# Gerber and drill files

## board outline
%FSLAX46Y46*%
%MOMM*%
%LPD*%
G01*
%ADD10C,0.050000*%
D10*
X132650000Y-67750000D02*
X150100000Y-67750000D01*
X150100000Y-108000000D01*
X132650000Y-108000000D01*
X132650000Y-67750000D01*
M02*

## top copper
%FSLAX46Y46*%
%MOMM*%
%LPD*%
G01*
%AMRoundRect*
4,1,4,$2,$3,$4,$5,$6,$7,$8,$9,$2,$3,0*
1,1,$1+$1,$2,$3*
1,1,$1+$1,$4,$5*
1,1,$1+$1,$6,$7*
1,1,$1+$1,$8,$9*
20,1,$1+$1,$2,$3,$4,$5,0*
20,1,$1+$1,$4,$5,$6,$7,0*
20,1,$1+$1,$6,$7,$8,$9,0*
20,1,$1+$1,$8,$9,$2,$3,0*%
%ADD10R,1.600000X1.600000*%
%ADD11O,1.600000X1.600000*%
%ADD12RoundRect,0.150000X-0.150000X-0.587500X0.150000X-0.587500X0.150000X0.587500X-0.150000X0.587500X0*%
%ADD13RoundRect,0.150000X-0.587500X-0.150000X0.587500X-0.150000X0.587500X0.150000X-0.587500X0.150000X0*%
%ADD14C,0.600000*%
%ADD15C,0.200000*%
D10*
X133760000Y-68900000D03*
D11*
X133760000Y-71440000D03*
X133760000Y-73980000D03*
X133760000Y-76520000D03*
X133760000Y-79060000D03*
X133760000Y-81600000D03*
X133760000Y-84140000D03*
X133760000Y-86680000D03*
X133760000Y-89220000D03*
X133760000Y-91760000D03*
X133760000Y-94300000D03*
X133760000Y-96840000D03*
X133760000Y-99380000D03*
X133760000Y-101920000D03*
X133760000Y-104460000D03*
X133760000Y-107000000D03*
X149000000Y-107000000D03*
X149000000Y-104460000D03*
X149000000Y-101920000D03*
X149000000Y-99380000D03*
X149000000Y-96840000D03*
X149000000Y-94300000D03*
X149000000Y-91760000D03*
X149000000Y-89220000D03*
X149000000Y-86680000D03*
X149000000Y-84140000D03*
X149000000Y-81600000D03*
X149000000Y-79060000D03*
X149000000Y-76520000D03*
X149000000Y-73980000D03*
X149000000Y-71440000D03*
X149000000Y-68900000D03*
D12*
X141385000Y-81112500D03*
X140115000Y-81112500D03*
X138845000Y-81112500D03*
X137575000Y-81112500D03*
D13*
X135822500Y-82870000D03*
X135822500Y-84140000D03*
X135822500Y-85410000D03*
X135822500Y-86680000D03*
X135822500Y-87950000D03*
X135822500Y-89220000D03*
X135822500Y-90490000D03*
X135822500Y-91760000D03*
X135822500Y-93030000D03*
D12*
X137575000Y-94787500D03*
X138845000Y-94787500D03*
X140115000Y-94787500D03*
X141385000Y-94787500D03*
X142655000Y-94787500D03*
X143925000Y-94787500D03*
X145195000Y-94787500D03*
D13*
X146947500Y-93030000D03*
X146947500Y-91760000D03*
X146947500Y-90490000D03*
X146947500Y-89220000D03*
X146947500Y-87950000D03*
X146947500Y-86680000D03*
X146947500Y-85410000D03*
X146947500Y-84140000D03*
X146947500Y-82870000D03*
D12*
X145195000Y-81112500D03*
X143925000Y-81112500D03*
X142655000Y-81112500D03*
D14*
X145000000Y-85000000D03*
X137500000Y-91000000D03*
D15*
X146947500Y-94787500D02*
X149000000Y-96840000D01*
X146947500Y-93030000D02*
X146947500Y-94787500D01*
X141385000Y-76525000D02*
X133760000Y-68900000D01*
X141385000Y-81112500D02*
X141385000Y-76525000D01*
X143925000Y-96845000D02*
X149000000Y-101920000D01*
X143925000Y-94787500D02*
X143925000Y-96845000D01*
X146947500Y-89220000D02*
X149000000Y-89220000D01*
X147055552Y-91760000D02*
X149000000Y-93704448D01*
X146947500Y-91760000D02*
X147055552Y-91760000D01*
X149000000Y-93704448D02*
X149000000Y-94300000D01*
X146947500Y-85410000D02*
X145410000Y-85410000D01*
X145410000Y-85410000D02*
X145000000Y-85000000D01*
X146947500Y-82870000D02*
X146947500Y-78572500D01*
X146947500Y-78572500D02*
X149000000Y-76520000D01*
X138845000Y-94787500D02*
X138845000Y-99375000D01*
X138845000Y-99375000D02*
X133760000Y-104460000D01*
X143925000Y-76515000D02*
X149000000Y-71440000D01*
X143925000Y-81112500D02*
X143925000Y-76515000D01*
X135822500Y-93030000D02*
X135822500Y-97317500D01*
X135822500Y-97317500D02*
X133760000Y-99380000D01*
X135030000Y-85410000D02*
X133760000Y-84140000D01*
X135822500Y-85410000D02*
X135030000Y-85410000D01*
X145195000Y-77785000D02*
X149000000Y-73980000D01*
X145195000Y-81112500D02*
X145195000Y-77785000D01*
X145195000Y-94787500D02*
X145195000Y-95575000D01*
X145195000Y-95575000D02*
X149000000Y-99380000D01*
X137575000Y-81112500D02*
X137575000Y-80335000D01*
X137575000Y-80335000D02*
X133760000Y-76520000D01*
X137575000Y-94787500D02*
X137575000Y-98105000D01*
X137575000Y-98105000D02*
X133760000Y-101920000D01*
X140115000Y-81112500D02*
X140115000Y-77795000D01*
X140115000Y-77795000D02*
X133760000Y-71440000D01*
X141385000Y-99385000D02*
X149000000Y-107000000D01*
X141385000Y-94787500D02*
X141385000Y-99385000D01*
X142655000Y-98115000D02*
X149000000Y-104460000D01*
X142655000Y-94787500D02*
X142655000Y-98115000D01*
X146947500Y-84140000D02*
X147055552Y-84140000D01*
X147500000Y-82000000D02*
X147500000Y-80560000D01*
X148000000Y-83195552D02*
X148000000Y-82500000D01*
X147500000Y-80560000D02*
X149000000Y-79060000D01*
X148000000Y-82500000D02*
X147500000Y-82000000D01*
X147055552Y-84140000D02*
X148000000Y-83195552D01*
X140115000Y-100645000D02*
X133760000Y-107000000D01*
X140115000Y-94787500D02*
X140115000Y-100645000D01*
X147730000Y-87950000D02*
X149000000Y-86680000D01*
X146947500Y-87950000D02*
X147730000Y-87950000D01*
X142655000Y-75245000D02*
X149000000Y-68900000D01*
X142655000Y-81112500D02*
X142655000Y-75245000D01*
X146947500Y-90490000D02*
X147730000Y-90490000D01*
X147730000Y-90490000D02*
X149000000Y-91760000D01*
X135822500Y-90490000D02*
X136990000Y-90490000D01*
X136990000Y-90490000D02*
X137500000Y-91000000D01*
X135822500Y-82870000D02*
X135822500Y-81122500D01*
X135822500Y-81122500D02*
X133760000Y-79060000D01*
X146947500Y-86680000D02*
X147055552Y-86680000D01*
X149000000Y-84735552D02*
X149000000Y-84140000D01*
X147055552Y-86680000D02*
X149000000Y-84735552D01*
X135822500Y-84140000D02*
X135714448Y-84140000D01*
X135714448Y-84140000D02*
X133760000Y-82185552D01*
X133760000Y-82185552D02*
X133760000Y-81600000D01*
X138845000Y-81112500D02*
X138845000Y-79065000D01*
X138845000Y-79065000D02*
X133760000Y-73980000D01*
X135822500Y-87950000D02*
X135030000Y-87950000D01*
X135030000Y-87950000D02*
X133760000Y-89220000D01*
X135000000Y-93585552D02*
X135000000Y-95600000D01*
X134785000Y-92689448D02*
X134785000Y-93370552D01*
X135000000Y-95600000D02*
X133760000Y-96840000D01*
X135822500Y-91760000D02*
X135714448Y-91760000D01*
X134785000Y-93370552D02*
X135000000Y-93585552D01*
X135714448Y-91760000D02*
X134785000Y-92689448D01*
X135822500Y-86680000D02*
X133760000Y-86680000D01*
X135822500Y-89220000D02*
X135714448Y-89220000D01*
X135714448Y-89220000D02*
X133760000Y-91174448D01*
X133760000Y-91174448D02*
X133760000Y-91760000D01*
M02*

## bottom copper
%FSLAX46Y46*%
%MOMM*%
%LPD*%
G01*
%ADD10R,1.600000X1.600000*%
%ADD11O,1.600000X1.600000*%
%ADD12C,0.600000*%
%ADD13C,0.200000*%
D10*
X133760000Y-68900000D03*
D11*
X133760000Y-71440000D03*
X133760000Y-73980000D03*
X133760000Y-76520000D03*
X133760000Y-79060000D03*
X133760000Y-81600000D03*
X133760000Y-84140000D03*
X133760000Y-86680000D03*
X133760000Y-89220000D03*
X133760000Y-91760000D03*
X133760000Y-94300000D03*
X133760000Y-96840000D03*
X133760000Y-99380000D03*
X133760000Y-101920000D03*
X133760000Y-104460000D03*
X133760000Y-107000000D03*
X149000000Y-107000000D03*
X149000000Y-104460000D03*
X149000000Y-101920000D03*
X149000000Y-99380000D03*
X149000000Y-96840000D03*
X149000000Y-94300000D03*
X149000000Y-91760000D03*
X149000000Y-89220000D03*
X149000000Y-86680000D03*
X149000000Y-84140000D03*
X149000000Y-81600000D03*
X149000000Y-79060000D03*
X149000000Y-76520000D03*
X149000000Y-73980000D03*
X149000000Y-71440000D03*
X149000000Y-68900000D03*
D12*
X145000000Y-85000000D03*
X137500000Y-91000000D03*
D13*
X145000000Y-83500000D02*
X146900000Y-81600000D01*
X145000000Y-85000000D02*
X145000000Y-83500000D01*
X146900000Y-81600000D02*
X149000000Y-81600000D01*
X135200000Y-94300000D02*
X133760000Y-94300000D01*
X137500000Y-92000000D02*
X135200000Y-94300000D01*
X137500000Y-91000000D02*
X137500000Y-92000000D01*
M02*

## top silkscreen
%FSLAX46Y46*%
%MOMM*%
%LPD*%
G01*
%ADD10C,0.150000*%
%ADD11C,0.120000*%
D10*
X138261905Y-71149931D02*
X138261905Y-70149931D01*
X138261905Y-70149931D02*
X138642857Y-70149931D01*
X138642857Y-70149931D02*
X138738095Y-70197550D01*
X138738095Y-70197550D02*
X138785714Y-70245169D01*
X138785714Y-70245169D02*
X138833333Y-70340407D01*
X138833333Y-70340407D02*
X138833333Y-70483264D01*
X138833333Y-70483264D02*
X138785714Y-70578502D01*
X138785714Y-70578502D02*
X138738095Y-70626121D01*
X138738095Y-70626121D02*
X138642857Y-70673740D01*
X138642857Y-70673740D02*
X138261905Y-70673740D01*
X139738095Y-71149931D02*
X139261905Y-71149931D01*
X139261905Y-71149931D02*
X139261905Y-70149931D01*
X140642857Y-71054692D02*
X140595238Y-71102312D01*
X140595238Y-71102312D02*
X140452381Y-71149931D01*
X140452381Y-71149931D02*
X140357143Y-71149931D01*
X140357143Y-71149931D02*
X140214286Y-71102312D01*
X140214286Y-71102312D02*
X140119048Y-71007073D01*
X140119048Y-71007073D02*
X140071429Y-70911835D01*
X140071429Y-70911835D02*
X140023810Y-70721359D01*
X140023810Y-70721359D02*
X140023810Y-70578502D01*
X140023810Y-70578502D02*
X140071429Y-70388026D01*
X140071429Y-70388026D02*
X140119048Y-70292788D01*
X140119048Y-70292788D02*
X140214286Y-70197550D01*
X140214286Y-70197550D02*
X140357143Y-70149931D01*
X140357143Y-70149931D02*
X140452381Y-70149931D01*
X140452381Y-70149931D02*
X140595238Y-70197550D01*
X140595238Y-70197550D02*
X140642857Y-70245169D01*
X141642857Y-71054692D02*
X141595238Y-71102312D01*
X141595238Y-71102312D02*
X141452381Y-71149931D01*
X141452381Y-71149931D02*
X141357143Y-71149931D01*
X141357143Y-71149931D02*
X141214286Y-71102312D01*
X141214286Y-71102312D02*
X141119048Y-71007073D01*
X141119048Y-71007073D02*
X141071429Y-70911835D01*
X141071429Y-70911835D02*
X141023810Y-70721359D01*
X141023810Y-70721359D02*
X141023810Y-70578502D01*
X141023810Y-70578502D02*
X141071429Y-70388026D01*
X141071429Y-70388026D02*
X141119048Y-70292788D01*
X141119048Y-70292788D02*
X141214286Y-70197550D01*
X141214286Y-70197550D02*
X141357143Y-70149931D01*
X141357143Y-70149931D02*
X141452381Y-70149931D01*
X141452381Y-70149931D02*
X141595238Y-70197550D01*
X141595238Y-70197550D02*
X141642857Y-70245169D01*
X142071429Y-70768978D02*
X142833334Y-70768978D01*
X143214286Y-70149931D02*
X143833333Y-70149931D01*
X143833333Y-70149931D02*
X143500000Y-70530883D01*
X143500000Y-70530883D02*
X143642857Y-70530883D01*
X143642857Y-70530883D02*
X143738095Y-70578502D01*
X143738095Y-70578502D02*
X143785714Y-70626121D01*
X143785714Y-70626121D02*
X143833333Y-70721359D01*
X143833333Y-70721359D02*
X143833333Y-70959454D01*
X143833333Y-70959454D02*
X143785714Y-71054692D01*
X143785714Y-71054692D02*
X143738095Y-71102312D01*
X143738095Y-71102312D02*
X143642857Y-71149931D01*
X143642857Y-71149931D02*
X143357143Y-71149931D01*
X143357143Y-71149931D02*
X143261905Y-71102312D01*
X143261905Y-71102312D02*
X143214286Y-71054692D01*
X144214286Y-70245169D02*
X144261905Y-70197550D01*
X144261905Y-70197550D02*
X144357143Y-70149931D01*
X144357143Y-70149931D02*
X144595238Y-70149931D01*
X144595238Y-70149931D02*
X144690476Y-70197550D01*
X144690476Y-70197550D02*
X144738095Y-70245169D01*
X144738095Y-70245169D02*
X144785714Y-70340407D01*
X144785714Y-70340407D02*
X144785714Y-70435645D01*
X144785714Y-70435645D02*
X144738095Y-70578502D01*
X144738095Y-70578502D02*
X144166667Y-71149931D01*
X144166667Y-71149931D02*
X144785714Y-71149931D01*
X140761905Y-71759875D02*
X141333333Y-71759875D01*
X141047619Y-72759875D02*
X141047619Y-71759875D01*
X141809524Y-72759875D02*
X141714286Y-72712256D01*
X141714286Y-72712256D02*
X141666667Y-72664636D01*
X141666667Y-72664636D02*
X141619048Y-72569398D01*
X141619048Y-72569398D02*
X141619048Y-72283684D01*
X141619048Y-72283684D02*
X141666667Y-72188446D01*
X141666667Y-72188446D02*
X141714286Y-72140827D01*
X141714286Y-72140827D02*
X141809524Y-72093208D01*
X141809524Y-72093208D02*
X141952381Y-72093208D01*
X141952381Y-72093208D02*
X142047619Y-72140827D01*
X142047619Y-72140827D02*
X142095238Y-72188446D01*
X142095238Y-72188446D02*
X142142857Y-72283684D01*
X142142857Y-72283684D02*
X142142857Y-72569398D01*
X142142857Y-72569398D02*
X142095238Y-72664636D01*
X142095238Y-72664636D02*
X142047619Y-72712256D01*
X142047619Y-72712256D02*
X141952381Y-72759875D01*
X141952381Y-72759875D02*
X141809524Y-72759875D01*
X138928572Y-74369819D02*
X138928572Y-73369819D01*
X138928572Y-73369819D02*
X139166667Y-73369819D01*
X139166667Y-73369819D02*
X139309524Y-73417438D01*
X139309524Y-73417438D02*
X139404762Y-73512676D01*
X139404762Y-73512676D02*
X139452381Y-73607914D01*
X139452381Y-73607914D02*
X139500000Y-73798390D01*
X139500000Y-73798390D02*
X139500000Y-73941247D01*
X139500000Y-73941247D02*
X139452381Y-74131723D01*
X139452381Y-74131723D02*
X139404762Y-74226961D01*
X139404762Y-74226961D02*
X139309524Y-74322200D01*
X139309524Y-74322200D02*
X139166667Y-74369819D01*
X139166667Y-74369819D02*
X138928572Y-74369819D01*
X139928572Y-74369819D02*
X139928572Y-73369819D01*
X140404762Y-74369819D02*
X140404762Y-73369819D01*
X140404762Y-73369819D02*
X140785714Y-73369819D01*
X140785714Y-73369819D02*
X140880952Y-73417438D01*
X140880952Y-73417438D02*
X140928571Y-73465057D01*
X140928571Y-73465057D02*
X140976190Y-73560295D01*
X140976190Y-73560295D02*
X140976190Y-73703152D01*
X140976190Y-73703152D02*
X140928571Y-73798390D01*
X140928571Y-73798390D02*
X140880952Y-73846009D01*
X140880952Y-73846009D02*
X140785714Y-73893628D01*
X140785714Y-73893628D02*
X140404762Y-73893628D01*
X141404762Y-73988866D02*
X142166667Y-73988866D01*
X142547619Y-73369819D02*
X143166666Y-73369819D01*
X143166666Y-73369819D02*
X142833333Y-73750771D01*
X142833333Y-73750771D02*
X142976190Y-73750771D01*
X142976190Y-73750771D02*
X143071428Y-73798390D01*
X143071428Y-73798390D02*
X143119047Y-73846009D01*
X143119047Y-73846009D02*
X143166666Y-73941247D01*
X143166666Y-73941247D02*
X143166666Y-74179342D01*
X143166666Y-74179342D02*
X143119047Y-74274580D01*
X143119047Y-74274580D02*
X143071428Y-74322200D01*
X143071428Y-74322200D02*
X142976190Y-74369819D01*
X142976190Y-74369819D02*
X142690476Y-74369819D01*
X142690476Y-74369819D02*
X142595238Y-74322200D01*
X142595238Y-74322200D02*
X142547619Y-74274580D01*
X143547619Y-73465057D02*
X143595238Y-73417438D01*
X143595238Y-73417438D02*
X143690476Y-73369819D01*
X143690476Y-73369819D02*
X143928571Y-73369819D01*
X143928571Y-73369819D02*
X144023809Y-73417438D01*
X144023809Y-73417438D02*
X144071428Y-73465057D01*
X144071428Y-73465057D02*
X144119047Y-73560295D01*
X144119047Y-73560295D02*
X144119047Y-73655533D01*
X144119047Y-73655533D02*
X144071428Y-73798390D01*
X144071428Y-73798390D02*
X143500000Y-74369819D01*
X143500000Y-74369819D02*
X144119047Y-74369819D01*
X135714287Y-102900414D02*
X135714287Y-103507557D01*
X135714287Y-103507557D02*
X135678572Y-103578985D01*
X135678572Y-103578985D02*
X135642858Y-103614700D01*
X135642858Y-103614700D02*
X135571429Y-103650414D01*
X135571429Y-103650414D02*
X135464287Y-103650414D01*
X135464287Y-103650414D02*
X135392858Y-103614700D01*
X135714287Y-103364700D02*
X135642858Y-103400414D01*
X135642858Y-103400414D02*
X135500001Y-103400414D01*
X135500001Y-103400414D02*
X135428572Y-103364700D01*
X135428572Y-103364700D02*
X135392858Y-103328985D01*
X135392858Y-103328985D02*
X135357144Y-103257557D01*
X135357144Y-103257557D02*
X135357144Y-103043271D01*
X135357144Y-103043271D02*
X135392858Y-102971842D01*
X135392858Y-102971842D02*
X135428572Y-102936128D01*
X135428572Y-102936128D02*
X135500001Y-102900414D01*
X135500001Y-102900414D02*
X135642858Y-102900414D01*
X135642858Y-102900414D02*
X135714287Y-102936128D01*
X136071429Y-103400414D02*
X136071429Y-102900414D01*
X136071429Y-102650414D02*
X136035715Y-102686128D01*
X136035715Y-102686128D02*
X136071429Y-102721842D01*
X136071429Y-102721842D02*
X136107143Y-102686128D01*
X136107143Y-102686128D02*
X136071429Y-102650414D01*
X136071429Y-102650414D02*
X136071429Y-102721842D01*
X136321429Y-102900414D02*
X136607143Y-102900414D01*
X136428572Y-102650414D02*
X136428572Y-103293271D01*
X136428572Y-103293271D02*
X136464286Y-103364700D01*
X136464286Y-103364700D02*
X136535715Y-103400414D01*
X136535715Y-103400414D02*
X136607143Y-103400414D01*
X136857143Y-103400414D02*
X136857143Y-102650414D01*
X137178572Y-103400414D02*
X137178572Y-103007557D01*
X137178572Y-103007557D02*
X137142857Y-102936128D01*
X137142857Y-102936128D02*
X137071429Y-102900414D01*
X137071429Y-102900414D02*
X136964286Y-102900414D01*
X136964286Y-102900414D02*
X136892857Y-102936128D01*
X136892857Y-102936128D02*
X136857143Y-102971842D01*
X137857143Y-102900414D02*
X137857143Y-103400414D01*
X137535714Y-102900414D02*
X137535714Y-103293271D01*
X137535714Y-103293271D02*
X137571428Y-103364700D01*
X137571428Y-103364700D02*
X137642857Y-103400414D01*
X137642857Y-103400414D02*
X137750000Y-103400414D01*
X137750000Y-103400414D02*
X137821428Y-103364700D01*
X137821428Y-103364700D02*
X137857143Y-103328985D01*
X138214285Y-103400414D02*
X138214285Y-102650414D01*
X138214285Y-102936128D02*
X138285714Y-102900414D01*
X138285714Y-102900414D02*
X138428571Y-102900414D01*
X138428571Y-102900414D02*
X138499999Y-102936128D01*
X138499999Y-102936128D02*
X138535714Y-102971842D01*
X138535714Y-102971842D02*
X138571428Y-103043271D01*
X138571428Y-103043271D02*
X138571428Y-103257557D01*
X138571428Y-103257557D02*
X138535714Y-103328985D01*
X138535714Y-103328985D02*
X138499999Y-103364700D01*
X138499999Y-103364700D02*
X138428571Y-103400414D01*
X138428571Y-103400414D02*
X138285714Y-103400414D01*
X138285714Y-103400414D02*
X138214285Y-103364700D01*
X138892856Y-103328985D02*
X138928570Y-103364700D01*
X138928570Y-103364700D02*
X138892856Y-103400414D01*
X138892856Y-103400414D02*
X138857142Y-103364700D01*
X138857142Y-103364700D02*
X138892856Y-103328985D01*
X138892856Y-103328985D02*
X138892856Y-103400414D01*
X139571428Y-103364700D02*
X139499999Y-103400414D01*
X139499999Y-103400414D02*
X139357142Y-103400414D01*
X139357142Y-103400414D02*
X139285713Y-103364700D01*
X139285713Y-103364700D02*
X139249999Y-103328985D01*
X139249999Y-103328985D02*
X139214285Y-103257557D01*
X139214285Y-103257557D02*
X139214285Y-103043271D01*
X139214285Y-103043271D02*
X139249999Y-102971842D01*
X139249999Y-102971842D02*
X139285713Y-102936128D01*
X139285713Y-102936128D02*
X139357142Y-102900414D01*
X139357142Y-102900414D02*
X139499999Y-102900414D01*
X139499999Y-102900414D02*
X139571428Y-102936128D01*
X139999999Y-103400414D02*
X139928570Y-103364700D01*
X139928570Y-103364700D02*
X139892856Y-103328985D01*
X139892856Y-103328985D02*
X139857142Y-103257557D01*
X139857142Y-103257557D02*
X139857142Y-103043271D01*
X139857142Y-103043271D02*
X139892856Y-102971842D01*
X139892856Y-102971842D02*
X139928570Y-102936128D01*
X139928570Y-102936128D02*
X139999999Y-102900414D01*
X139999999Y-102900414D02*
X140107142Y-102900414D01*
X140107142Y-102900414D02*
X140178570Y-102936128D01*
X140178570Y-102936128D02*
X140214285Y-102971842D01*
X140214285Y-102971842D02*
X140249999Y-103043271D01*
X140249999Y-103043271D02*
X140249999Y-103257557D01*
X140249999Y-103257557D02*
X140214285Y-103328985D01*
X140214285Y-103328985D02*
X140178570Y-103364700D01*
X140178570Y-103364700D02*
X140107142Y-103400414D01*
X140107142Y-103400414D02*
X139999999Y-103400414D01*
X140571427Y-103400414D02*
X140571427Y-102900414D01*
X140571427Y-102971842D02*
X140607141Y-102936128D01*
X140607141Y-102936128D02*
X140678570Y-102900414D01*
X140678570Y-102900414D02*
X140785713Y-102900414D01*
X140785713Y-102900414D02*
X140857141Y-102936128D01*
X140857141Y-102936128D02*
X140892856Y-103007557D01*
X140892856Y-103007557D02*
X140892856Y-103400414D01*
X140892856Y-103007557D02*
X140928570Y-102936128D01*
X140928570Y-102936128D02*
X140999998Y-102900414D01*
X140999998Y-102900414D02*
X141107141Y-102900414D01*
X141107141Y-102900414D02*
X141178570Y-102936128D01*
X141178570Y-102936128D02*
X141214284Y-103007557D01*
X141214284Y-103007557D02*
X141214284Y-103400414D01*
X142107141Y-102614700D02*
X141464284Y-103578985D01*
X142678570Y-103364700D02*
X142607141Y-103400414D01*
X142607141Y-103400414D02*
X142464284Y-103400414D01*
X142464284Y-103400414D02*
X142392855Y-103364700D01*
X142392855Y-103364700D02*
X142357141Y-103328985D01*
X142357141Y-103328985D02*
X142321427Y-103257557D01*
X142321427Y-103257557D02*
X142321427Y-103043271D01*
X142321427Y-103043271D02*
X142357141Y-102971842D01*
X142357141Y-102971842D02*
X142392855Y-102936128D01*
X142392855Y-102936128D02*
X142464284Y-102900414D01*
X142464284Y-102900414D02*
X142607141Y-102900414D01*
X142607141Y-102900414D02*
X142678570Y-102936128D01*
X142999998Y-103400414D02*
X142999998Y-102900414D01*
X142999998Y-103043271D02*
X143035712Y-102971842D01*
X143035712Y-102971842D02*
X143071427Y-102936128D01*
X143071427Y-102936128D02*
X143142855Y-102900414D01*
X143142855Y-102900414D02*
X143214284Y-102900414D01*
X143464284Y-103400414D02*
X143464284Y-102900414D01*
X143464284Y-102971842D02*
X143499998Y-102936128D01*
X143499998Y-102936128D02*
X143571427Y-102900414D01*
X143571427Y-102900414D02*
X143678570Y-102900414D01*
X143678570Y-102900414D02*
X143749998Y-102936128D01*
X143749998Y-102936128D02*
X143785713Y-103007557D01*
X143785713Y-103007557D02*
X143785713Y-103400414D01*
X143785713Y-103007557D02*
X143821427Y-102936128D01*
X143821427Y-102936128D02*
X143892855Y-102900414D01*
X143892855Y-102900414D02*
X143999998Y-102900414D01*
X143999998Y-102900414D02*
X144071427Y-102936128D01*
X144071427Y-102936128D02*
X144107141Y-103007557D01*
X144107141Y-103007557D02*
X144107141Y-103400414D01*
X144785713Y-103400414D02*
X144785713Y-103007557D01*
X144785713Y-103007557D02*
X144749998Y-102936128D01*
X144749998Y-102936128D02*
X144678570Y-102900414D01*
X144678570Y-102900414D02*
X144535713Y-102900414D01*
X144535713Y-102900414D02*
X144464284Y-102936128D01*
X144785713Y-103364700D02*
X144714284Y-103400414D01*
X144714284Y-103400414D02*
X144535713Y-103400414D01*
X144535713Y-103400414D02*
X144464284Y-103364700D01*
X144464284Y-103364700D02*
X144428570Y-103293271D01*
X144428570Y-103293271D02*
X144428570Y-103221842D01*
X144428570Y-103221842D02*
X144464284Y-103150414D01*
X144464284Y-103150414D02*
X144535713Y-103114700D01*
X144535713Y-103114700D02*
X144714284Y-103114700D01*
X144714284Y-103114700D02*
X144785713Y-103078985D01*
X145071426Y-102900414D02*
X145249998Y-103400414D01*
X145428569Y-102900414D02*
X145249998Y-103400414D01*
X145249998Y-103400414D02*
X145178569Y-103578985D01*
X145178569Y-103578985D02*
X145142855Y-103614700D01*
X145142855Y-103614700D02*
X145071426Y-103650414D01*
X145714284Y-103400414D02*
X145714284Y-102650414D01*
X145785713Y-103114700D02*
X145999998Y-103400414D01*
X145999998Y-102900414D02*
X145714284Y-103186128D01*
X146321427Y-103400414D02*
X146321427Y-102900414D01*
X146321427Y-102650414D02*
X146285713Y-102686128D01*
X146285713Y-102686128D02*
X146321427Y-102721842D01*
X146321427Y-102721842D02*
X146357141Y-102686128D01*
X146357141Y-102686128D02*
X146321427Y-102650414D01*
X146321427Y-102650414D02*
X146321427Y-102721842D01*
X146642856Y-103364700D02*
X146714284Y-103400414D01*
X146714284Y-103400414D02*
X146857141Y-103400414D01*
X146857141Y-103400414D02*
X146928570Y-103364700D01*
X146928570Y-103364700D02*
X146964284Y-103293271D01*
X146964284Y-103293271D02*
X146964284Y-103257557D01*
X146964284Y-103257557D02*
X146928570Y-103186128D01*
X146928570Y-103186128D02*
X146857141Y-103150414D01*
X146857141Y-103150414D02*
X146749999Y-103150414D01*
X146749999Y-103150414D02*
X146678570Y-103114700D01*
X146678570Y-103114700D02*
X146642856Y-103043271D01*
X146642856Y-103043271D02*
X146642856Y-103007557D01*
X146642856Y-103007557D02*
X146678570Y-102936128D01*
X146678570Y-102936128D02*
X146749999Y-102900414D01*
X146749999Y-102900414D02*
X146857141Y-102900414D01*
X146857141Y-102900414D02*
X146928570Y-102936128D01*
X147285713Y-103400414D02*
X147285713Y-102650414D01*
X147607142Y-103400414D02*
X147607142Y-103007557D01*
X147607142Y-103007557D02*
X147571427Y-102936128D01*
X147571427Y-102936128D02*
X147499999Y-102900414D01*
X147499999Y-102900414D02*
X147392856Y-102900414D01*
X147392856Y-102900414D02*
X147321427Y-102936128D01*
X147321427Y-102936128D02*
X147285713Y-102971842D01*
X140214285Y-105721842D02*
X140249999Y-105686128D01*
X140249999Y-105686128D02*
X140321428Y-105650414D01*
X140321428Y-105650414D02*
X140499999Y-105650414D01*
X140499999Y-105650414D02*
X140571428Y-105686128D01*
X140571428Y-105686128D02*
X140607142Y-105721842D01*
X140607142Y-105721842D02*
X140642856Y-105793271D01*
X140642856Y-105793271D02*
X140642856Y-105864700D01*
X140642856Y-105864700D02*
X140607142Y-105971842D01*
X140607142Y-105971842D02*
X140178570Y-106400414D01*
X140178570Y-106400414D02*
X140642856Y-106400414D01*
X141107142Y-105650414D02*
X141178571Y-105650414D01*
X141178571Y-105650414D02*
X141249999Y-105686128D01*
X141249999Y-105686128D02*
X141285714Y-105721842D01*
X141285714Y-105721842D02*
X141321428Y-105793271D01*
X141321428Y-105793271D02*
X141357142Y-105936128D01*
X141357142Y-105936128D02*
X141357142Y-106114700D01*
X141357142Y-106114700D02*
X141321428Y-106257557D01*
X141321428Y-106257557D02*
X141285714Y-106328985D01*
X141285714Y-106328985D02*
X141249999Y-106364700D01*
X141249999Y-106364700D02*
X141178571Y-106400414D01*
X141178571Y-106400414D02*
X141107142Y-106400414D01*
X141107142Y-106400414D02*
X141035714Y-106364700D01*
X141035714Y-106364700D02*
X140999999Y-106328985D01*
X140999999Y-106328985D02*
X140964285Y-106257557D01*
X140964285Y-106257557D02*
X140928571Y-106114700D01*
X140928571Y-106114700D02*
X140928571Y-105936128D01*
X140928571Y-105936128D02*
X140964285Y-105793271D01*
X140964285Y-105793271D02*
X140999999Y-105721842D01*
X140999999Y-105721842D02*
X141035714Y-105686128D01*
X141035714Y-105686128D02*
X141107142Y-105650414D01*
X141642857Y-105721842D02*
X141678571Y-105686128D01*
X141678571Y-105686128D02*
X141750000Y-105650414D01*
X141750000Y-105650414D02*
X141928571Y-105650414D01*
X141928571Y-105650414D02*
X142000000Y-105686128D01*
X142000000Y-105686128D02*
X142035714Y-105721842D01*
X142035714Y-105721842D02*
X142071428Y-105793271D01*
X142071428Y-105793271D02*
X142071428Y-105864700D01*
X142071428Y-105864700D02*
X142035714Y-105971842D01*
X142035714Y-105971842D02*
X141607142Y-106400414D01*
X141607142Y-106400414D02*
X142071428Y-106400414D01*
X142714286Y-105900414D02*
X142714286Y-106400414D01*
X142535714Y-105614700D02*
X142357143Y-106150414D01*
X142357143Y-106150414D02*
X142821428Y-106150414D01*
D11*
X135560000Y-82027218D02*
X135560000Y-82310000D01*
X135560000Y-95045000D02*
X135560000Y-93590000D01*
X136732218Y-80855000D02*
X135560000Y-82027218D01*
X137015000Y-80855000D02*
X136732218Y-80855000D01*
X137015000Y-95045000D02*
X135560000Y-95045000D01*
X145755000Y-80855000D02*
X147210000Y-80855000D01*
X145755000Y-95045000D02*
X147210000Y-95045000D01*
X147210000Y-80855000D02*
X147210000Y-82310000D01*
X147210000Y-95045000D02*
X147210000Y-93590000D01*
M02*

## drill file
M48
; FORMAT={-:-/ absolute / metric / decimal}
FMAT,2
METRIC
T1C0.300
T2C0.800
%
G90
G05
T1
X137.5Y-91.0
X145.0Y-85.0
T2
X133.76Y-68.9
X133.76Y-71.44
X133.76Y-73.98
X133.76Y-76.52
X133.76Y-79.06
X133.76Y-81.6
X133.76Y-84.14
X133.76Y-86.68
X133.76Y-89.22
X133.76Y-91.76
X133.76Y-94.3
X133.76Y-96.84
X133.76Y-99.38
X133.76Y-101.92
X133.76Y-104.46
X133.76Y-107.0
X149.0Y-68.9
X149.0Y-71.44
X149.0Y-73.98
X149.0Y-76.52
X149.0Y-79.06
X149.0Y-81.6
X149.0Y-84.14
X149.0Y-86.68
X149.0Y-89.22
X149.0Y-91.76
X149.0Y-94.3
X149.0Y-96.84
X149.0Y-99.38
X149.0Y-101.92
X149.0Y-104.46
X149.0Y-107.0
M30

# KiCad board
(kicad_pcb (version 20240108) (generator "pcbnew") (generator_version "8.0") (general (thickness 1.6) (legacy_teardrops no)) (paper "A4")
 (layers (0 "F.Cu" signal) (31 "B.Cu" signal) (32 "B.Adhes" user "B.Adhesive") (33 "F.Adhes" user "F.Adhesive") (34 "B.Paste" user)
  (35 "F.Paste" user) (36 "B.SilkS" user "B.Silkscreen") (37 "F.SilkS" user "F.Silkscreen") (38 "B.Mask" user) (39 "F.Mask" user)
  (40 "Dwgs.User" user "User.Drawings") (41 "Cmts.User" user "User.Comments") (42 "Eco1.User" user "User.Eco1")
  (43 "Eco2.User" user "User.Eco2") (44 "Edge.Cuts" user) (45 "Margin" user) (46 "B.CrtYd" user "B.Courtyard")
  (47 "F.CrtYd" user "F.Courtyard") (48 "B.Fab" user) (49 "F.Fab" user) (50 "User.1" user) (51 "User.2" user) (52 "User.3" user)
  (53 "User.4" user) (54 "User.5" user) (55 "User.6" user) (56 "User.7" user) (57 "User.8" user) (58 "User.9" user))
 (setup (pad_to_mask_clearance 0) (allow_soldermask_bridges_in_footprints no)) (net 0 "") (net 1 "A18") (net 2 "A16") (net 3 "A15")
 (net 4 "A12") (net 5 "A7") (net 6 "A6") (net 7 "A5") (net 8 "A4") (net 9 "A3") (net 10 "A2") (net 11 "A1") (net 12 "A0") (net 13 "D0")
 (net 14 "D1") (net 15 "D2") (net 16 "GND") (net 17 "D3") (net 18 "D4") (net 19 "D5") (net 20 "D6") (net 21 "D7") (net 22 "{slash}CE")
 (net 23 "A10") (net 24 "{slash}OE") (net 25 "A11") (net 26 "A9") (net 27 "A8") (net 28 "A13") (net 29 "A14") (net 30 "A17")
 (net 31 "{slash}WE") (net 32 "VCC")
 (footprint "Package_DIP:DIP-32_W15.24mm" (layer "F.Cu") (at 133.76 68.9)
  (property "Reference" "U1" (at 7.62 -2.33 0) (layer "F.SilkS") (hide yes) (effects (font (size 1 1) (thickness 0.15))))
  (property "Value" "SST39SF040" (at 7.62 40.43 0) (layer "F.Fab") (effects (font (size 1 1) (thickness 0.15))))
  (pad "1" thru_hole rect (at 0 0) (size 1.6 1.6) (drill 0.8) (layers "*.Cu" "*.Mask") (remove_unused_layers no) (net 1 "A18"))
  (pad "2" thru_hole oval (at 0 2.54) (size 1.6 1.6) (drill 0.8) (layers "*.Cu" "*.Mask") (remove_unused_layers no) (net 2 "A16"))
  (pad "3" thru_hole oval (at 0 5.08) (size 1.6 1.6) (drill 0.8) (layers "*.Cu" "*.Mask") (remove_unused_layers no) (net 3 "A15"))
  (pad "4" thru_hole oval (at 0 7.62) (size 1.6 1.6) (drill 0.8) (layers "*.Cu" "*.Mask") (remove_unused_layers no) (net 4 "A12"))
  (pad "5" thru_hole oval (at 0 10.16) (size 1.6 1.6) (drill 0.8) (layers "*.Cu" "*.Mask") (remove_unused_layers no) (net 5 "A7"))
  (pad "6" thru_hole oval (at 0 12.7) (size 1.6 1.6) (drill 0.8) (layers "*.Cu" "*.Mask") (remove_unused_layers no) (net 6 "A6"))
  (pad "7" thru_hole oval (at 0 15.24) (size 1.6 1.6) (drill 0.8) (layers "*.Cu" "*.Mask") (remove_unused_layers no) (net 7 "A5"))
  (pad "8" thru_hole oval (at 0 17.78) (size 1.6 1.6) (drill 0.8) (layers "*.Cu" "*.Mask") (remove_unused_layers no) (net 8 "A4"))
  (pad "9" thru_hole oval (at 0 20.32) (size 1.6 1.6) (drill 0.8) (layers "*.Cu" "*.Mask") (remove_unused_layers no) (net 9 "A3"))
  (pad "10" thru_hole oval (at 0 22.86) (size 1.6 1.6) (drill 0.8) (layers "*.Cu" "*.Mask") (remove_unused_layers no) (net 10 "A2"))
  (pad "11" thru_hole oval (at 0 25.4) (size 1.6 1.6) (drill 0.8) (layers "*.Cu" "*.Mask") (remove_unused_layers no) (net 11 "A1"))
  (pad "12" thru_hole oval (at 0 27.94) (size 1.6 1.6) (drill 0.8) (layers "*.Cu" "*.Mask") (remove_unused_layers no) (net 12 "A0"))
  (pad "13" thru_hole oval (at 0 30.48) (size 1.6 1.6) (drill 0.8) (layers "*.Cu" "*.Mask") (remove_unused_layers no) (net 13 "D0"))
  (pad "14" thru_hole oval (at 0 33.02) (size 1.6 1.6) (drill 0.8) (layers "*.Cu" "*.Mask") (remove_unused_layers no) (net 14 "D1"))
  (pad "15" thru_hole oval (at 0 35.56) (size 1.6 1.6) (drill 0.8) (layers "*.Cu" "*.Mask") (remove_unused_layers no) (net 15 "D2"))
  (pad "16" thru_hole oval (at 0 38.1) (size 1.6 1.6) (drill 0.8) (layers "*.Cu" "*.Mask") (remove_unused_layers no) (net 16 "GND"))
  (pad "17" thru_hole oval (at 15.24 38.1) (size 1.6 1.6) (drill 0.8) (layers "*.Cu" "*.Mask") (remove_unused_layers no) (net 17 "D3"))
  (pad "18" thru_hole oval (at 15.24 35.56) (size 1.6 1.6) (drill 0.8) (layers "*.Cu" "*.Mask") (remove_unused_layers no) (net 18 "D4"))
  (pad "19" thru_hole oval (at 15.24 33.02) (size 1.6 1.6) (drill 0.8) (layers "*.Cu" "*.Mask") (remove_unused_layers no) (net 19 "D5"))
  (pad "20" thru_hole oval (at 15.24 30.48) (size 1.6 1.6) (drill 0.8) (layers "*.Cu" "*.Mask") (remove_unused_layers no) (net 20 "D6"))
  (pad "21" thru_hole oval (at 15.24 27.94) (size 1.6 1.6) (drill 0.8) (layers "*.Cu" "*.Mask") (remove_unused_layers no) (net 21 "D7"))
  (pad "22" thru_hole oval (at 15.24 25.4) (size 1.6 1.6) (drill 0.8) (layers "*.Cu" "*.Mask") (remove_unused_layers no)
   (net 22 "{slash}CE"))
  (pad "23" thru_hole oval (at 15.24 22.86) (size 1.6 1.6) (drill 0.8) (layers "*.Cu" "*.Mask") (remove_unused_layers no) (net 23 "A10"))
  (pad "24" thru_hole oval (at 15.24 20.32) (size 1.6 1.6) (drill 0.8) (layers "*.Cu" "*.Mask") (remove_unused_layers no)
   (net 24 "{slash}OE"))
  (pad "25" thru_hole oval (at 15.24 17.78) (size 1.6 1.6) (drill 0.8) (layers "*.Cu" "*.Mask") (remove_unused_layers no) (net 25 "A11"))
  (pad "26" thru_hole oval (at 15.24 15.24) (size 1.6 1.6) (drill 0.8) (layers "*.Cu" "*.Mask") (remove_unused_layers no) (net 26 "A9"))
  (pad "27" thru_hole oval (at 15.24 12.7) (size 1.6 1.6) (drill 0.8) (layers "*.Cu" "*.Mask") (remove_unused_layers no) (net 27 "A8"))
  (pad "28" thru_hole oval (at 15.24 10.16) (size 1.6 1.6) (drill 0.8) (layers "*.Cu" "*.Mask") (remove_unused_layers no) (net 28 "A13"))
  (pad "29" thru_hole oval (at 15.24 7.62) (size 1.6 1.6) (drill 0.8) (layers "*.Cu" "*.Mask") (remove_unused_layers no) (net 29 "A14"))
  (pad "30" thru_hole oval (at 15.24 5.08) (size 1.6 1.6) (drill 0.8) (layers "*.Cu" "*.Mask") (remove_unused_layers no) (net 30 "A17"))
  (pad "31" thru_hole oval (at 15.24 2.54) (size 1.6 1.6) (drill 0.8) (layers "*.Cu" "*.Mask") (remove_unused_layers no)
   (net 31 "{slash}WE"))
  (pad "32" thru_hole oval (at 15.24 0) (size 1.6 1.6) (drill 0.8) (layers "*.Cu" "*.Mask") (remove_unused_layers no) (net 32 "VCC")))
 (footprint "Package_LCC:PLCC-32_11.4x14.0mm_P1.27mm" (layer "F.Cu") (at 141.385 87.95)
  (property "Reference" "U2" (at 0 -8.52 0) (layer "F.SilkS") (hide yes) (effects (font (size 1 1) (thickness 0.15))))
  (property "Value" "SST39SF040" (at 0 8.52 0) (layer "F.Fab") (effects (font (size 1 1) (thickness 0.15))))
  (fp_line (start -5.825 -5.922782) (end -5.825 -5.64) (stroke (width 0.12) (type solid)) (layer "F.SilkS"))
  (fp_line (start -5.825 7.095) (end -5.825 5.64) (stroke (width 0.12) (type solid)) (layer "F.SilkS"))
  (fp_line (start -4.652782 -7.095) (end -5.825 -5.922782) (stroke (width 0.12) (type solid)) (layer "F.SilkS"))
  (fp_line (start -4.37 -7.095) (end -4.652782 -7.095) (stroke (width 0.12) (type solid)) (layer "F.SilkS"))
  (fp_line (start -4.37 7.095) (end -5.825 7.095) (stroke (width 0.12) (type solid)) (layer "F.SilkS"))
  (fp_line (start 4.37 -7.095) (end 5.825 -7.095) (stroke (width 0.12) (type solid)) (layer "F.SilkS"))
  (fp_line (start 4.37 7.095) (end 5.825 7.095) (stroke (width 0.12) (type solid)) (layer "F.SilkS"))
  (fp_line (start 5.825 -7.095) (end 5.825 -5.64) (stroke (width 0.12) (type solid)) (layer "F.SilkS"))
  (fp_line (start 5.825 7.095) (end 5.825 5.64) (stroke (width 0.12) (type solid)) (layer "F.SilkS"))
  (pad "1" smd roundrect (at 0 -6.8375) (size 0.6 1.475) (layers "F.Cu" "F.Paste" "F.Mask") (roundrect_rratio 0.25) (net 1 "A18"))
  (pad "2" smd roundrect (at -1.27 -6.8375) (size 0.6 1.475) (layers "F.Cu" "F.Paste" "F.Mask") (roundrect_rratio 0.25) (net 2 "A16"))
  (pad "3" smd roundrect (at -2.54 -6.8375) (size 0.6 1.475) (layers "F.Cu" "F.Paste" "F.Mask") (roundrect_rratio 0.25) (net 3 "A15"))
  (pad "4" smd roundrect (at -3.81 -6.8375) (size 0.6 1.475) (layers "F.Cu" "F.Paste" "F.Mask") (roundrect_rratio 0.25) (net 4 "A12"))
  (pad "5" smd roundrect (at -5.5625 -5.08) (size 1.475 0.6) (layers "F.Cu" "F.Paste" "F.Mask") (roundrect_rratio 0.25) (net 5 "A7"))
  (pad "6" smd roundrect (at -5.5625 -3.81) (size 1.475 0.6) (layers "F.Cu" "F.Paste" "F.Mask") (roundrect_rratio 0.25) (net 6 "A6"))
  (pad "7" smd roundrect (at -5.5625 -2.54) (size 1.475 0.6) (layers "F.Cu" "F.Paste" "F.Mask") (roundrect_rratio 0.25) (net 7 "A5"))
  (pad "8" smd roundrect (at -5.5625 -1.27) (size 1.475 0.6) (layers "F.Cu" "F.Paste" "F.Mask") (roundrect_rratio 0.25) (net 8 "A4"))
  (pad "9" smd roundrect (at -5.5625 0) (size 1.475 0.6) (layers "F.Cu" "F.Paste" "F.Mask") (roundrect_rratio 0.25) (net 9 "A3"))
  (pad "10" smd roundrect (at -5.5625 1.27) (size 1.475 0.6) (layers "F.Cu" "F.Paste" "F.Mask") (roundrect_rratio 0.25) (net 10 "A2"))
  (pad "11" smd roundrect (at -5.5625 2.54) (size 1.475 0.6) (layers "F.Cu" "F.Paste" "F.Mask") (roundrect_rratio 0.25) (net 11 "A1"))
  (pad "12" smd roundrect (at -5.5625 3.81) (size 1.475 0.6) (layers "F.Cu" "F.Paste" "F.Mask") (roundrect_rratio 0.25) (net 12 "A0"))
  (pad "13" smd roundrect (at -5.5625 5.08) (size 1.475 0.6) (layers "F.Cu" "F.Paste" "F.Mask") (roundrect_rratio 0.25) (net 13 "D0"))
  (pad "14" smd roundrect (at -3.81 6.8375) (size 0.6 1.475) (layers "F.Cu" "F.Paste" "F.Mask") (roundrect_rratio 0.25) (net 14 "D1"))
  (pad "15" smd roundrect (at -2.54 6.8375) (size 0.6 1.475) (layers "F.Cu" "F.Paste" "F.Mask") (roundrect_rratio 0.25) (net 15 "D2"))
  (pad "16" smd roundrect (at -1.27 6.8375) (size 0.6 1.475) (layers "F.Cu" "F.Paste" "F.Mask") (roundrect_rratio 0.25) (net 16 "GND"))
  (pad "17" smd roundrect (at 0 6.8375) (size 0.6 1.475) (layers "F.Cu" "F.Paste" "F.Mask") (roundrect_rratio 0.25) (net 17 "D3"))
  (pad "18" smd roundrect (at 1.27 6.8375) (size 0.6 1.475) (layers "F.Cu" "F.Paste" "F.Mask") (roundrect_rratio 0.25) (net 18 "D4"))
  (pad "19" smd roundrect (at 2.54 6.8375) (size 0.6 1.475) (layers "F.Cu" "F.Paste" "F.Mask") (roundrect_rratio 0.25) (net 19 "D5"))
  (pad "20" smd roundrect (at 3.81 6.8375) (size 0.6 1.475) (layers "F.Cu" "F.Paste" "F.Mask") (roundrect_rratio 0.25) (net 20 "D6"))
  (pad "21" smd roundrect (at 5.5625 5.08) (size 1.475 0.6) (layers "F.Cu" "F.Paste" "F.Mask") (roundrect_rratio 0.25) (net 21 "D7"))
  (pad "22" smd roundrect (at 5.5625 3.81) (size 1.475 0.6) (layers "F.Cu" "F.Paste" "F.Mask") (roundrect_rratio 0.25) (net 22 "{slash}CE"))
  (pad "23" smd roundrect (at 5.5625 2.54) (size 1.475 0.6) (layers "F.Cu" "F.Paste" "F.Mask") (roundrect_rratio 0.25) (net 23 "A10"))
  (pad "24" smd roundrect (at 5.5625 1.27) (size 1.475 0.6) (layers "F.Cu" "F.Paste" "F.Mask") (roundrect_rratio 0.25) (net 24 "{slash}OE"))
  (pad "25" smd roundrect (at 5.5625 0) (size 1.475 0.6) (layers "F.Cu" "F.Paste" "F.Mask") (roundrect_rratio 0.25) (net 25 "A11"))
  (pad "26" smd roundrect (at 5.5625 -1.27) (size 1.475 0.6) (layers "F.Cu" "F.Paste" "F.Mask") (roundrect_rratio 0.25) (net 26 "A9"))
  (pad "27" smd roundrect (at 5.5625 -2.54) (size 1.475 0.6) (layers "F.Cu" "F.Paste" "F.Mask") (roundrect_rratio 0.25) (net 27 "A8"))
  (pad "28" smd roundrect (at 5.5625 -3.81) (size 1.475 0.6) (layers "F.Cu" "F.Paste" "F.Mask") (roundrect_rratio 0.25) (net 28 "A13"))
  (pad "29" smd roundrect (at 5.5625 -5.08) (size 1.475 0.6) (layers "F.Cu" "F.Paste" "F.Mask") (roundrect_rratio 0.25) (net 29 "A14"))
  (pad "30" smd roundrect (at 3.81 -6.8375) (size 0.6 1.475) (layers "F.Cu" "F.Paste" "F.Mask") (roundrect_rratio 0.25) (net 30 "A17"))
  (pad "31" smd roundrect (at 2.54 -6.8375) (size 0.6 1.475) (layers "F.Cu" "F.Paste" "F.Mask") (roundrect_rratio 0.25) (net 31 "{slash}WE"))
  (pad "32" smd roundrect (at 1.27 -6.8375) (size 0.6 1.475) (layers "F.Cu" "F.Paste" "F.Mask") (roundrect_rratio 0.25) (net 32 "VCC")))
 (gr_rect (start 132.65 67.75) (end 150.1 108) (stroke (width 0.05) (type default)) (fill none) (layer "Edge.Cuts"))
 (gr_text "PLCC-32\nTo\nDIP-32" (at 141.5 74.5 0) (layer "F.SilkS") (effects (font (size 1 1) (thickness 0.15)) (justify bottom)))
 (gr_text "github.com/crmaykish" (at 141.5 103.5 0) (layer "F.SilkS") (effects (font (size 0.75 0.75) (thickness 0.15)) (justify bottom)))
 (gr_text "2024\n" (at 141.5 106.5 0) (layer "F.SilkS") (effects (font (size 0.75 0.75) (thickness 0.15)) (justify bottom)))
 (segment (start 146.9475 94.7875) (end 149 96.84) (width 0.2) (layer "F.Cu") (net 21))
 (segment (start 146.9475 93.03) (end 146.9475 94.7875) (width 0.2) (layer "F.Cu") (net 21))
 (segment (start 141.385 76.525) (end 133.76 68.9) (width 0.2) (layer "F.Cu") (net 1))
 (segment (start 141.385 81.1125) (end 141.385 76.525) (width 0.2) (layer "F.Cu") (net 1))
 (segment (start 143.925 96.845) (end 149 101.92) (width 0.2) (layer "F.Cu") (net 19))
 (segment (start 143.925 94.7875) (end 143.925 96.845) (width 0.2) (layer "F.Cu") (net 19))
 (segment (start 146.9475 89.22) (end 149 89.22) (width 0.2) (layer "F.Cu") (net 24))
 (segment (start 147.055552 91.76) (end 149 93.704448) (width 0.2) (layer "F.Cu") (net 22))
 (segment (start 146.9475 91.76) (end 147.055552 91.76) (width 0.2) (layer "F.Cu") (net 22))
 (segment (start 149 93.704448) (end 149 94.3) (width 0.2) (layer "F.Cu") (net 22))
 (segment (start 146.9475 85.41) (end 145.41 85.41) (width 0.2) (layer "F.Cu") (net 27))
 (segment (start 145.41 85.41) (end 145 85) (width 0.2) (layer "F.Cu") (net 27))
 (via (at 145 85) (size 0.6) (drill 0.3) (layers "F.Cu" "B.Cu") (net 27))
 (segment (start 145 83.5) (end 146.9 81.6) (width 0.2) (layer "B.Cu") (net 27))
 (segment (start 145 85) (end 145 83.5) (width 0.2) (layer "B.Cu") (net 27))
 (segment (start 146.9 81.6) (end 149 81.6) (width 0.2) (layer "B.Cu") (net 27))
 (segment (start 146.9475 82.87) (end 146.9475 78.5725) (width 0.2) (layer "F.Cu") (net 29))
 (segment (start 146.9475 78.5725) (end 149 76.52) (width 0.2) (layer "F.Cu") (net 29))
 (segment (start 138.845 94.7875) (end 138.845 99.375) (width 0.2) (layer "F.Cu") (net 15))
 (segment (start 138.845 99.375) (end 133.76 104.46) (width 0.2) (layer "F.Cu") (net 15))
 (segment (start 143.925 76.515) (end 149 71.44) (width 0.2) (layer "F.Cu") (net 31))
 (segment (start 143.925 81.1125) (end 143.925 76.515) (width 0.2) (layer "F.Cu") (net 31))
 (segment (start 135.8225 93.03) (end 135.8225 97.3175) (width 0.2) (layer "F.Cu") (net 13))
 (segment (start 135.8225 97.3175) (end 133.76 99.38) (width 0.2) (layer "F.Cu") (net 13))
 (segment (start 135.03 85.41) (end 133.76 84.14) (width 0.2) (layer "F.Cu") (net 7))
 (segment (start 135.8225 85.41) (end 135.03 85.41) (width 0.2) (layer "F.Cu") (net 7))
 (segment (start 145.195 77.785) (end 149 73.98) (width 0.2) (layer "F.Cu") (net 30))
 (segment (start 145.195 81.1125) (end 145.195 77.785) (width 0.2) (layer "F.Cu") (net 30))
 (segment (start 145.195 94.7875) (end 145.195 95.575) (width 0.2) (layer "F.Cu") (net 20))
 (segment (start 145.195 95.575) (end 149 99.38) (width 0.2) (layer "F.Cu") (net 20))
 (segment (start 137.575 81.1125) (end 137.575 80.335) (width 0.2) (layer "F.Cu") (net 4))
 (segment (start 137.575 80.335) (end 133.76 76.52) (width 0.2) (layer "F.Cu") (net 4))
 (segment (start 137.575 94.7875) (end 137.575 98.105) (width 0.2) (layer "F.Cu") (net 14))
 (segment (start 137.575 98.105) (end 133.76 101.92) (width 0.2) (layer "F.Cu") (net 14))
 (segment (start 140.115 81.1125) (end 140.115 77.795) (width 0.2) (layer "F.Cu") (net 2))
 (segment (start 140.115 77.795) (end 133.76 71.44) (width 0.2) (layer "F.Cu") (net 2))
 (segment (start 141.385 99.385) (end 149 107) (width 0.2) (layer "F.Cu") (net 17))
 (segment (start 141.385 94.7875) (end 141.385 99.385) (width 0.2) (layer "F.Cu") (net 17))
 (segment (start 142.655 98.115) (end 149 104.46) (width 0.2) (layer "F.Cu") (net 18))
 (segment (start 142.655 94.7875) (end 142.655 98.115) (width 0.2) (layer "F.Cu") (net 18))
 (segment (start 146.9475 84.14) (end 147.055552 84.14) (width 0.2) (layer "F.Cu") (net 28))
 (segment (start 147.5 82) (end 147.5 80.56) (width 0.2) (layer "F.Cu") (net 28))
 (segment (start 148 83.195552) (end 148 82.5) (width 0.2) (layer "F.Cu") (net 28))
 (segment (start 147.5 80.56) (end 149 79.06) (width 0.2) (layer "F.Cu") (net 28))
 (segment (start 148 82.5) (end 147.5 82) (width 0.2) (layer "F.Cu") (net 28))
 (segment (start 147.055552 84.14) (end 148 83.195552) (width 0.2) (layer "F.Cu") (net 28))
 (segment (start 140.115 100.645) (end 133.76 107) (width 0.2) (layer "F.Cu") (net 16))
 (segment (start 140.115 94.7875) (end 140.115 100.645) (width 0.2) (layer "F.Cu") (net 16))
 (segment (start 147.73 87.95) (end 149 86.68) (width 0.2) (layer "F.Cu") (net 25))
 (segment (start 146.9475 87.95) (end 147.73 87.95) (width 0.2) (layer "F.Cu") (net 25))
 (segment (start 142.655 75.245) (end 149 68.9) (width 0.2) (layer "F.Cu") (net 32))
 (segment (start 142.655 81.1125) (end 142.655 75.245) (width 0.2) (layer "F.Cu") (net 32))
 (segment (start 146.9475 90.49) (end 147.73 90.49) (width 0.2) (layer "F.Cu") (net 23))
 (segment (start 147.73 90.49) (end 149 91.76) (width 0.2) (layer "F.Cu") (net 23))
 (segment (start 135.8225 90.49) (end 136.99 90.49) (width 0.2) (layer "F.Cu") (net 11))
 (segment (start 136.99 90.49) (end 137.5 91) (width 0.2) (layer "F.Cu") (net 11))
 (via (at 137.5 91) (size 0.6) (drill 0.3) (layers "F.Cu" "B.Cu") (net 11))
 (segment (start 135.2 94.3) (end 133.76 94.3) (width 0.2) (layer "B.Cu") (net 11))
 (segment (start 137.5 92) (end 135.2 94.3) (width 0.2) (layer "B.Cu") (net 11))
 (segment (start 137.5 91) (end 137.5 92) (width 0.2) (layer "B.Cu") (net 11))
 (segment (start 135.8225 82.87) (end 135.8225 81.1225) (width 0.2) (layer "F.Cu") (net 5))
 (segment (start 135.8225 81.1225) (end 133.76 79.06) (width 0.2) (layer "F.Cu") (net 5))
 (segment (start 146.9475 86.68) (end 147.055552 86.68) (width 0.2) (layer "F.Cu") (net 26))
 (segment (start 149 84.735552) (end 149 84.14) (width 0.2) (layer "F.Cu") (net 26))
 (segment (start 147.055552 86.68) (end 149 84.735552) (width 0.2) (layer "F.Cu") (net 26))
 (segment (start 135.8225 84.14) (end 135.714448 84.14) (width 0.2) (layer "F.Cu") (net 6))
 (segment (start 135.714448 84.14) (end 133.76 82.185552) (width 0.2) (layer "F.Cu") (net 6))
 (segment (start 133.76 82.185552) (end 133.76 81.6) (width 0.2) (layer "F.Cu") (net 6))
 (segment (start 138.845 81.1125) (end 138.845 79.065) (width 0.2) (layer "F.Cu") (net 3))
 (segment (start 138.845 79.065) (end 133.76 73.98) (width 0.2) (layer "F.Cu") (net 3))
 (segment (start 135.8225 87.95) (end 135.03 87.95) (width 0.2) (layer "F.Cu") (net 9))
 (segment (start 135.03 87.95) (end 133.76 89.22) (width 0.2) (layer "F.Cu") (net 9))
 (segment (start 135 93.585552) (end 135 95.6) (width 0.2) (layer "F.Cu") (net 12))
 (segment (start 134.785 92.689448) (end 134.785 93.370552) (width 0.2) (layer "F.Cu") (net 12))
 (segment (start 135 95.6) (end 133.76 96.84) (width 0.2) (layer "F.Cu") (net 12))
 (segment (start 135.8225 91.76) (end 135.714448 91.76) (width 0.2) (layer "F.Cu") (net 12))
 (segment (start 134.785 93.370552) (end 135 93.585552) (width 0.2) (layer "F.Cu") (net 12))
 (segment (start 135.714448 91.76) (end 134.785 92.689448) (width 0.2) (layer "F.Cu") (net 12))
 (segment (start 135.8225 86.68) (end 133.76 86.68) (width 0.2) (layer "F.Cu") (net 8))
 (segment (start 135.8225 89.22) (end 135.714448 89.22) (width 0.2) (layer "F.Cu") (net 10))
 (segment (start 135.714448 89.22) (end 133.76 91.174448) (width 0.2) (layer "F.Cu") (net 10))
 (segment (start 133.76 91.174448) (end 133.76 91.76) (width 0.2) (layer "F.Cu") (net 10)))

